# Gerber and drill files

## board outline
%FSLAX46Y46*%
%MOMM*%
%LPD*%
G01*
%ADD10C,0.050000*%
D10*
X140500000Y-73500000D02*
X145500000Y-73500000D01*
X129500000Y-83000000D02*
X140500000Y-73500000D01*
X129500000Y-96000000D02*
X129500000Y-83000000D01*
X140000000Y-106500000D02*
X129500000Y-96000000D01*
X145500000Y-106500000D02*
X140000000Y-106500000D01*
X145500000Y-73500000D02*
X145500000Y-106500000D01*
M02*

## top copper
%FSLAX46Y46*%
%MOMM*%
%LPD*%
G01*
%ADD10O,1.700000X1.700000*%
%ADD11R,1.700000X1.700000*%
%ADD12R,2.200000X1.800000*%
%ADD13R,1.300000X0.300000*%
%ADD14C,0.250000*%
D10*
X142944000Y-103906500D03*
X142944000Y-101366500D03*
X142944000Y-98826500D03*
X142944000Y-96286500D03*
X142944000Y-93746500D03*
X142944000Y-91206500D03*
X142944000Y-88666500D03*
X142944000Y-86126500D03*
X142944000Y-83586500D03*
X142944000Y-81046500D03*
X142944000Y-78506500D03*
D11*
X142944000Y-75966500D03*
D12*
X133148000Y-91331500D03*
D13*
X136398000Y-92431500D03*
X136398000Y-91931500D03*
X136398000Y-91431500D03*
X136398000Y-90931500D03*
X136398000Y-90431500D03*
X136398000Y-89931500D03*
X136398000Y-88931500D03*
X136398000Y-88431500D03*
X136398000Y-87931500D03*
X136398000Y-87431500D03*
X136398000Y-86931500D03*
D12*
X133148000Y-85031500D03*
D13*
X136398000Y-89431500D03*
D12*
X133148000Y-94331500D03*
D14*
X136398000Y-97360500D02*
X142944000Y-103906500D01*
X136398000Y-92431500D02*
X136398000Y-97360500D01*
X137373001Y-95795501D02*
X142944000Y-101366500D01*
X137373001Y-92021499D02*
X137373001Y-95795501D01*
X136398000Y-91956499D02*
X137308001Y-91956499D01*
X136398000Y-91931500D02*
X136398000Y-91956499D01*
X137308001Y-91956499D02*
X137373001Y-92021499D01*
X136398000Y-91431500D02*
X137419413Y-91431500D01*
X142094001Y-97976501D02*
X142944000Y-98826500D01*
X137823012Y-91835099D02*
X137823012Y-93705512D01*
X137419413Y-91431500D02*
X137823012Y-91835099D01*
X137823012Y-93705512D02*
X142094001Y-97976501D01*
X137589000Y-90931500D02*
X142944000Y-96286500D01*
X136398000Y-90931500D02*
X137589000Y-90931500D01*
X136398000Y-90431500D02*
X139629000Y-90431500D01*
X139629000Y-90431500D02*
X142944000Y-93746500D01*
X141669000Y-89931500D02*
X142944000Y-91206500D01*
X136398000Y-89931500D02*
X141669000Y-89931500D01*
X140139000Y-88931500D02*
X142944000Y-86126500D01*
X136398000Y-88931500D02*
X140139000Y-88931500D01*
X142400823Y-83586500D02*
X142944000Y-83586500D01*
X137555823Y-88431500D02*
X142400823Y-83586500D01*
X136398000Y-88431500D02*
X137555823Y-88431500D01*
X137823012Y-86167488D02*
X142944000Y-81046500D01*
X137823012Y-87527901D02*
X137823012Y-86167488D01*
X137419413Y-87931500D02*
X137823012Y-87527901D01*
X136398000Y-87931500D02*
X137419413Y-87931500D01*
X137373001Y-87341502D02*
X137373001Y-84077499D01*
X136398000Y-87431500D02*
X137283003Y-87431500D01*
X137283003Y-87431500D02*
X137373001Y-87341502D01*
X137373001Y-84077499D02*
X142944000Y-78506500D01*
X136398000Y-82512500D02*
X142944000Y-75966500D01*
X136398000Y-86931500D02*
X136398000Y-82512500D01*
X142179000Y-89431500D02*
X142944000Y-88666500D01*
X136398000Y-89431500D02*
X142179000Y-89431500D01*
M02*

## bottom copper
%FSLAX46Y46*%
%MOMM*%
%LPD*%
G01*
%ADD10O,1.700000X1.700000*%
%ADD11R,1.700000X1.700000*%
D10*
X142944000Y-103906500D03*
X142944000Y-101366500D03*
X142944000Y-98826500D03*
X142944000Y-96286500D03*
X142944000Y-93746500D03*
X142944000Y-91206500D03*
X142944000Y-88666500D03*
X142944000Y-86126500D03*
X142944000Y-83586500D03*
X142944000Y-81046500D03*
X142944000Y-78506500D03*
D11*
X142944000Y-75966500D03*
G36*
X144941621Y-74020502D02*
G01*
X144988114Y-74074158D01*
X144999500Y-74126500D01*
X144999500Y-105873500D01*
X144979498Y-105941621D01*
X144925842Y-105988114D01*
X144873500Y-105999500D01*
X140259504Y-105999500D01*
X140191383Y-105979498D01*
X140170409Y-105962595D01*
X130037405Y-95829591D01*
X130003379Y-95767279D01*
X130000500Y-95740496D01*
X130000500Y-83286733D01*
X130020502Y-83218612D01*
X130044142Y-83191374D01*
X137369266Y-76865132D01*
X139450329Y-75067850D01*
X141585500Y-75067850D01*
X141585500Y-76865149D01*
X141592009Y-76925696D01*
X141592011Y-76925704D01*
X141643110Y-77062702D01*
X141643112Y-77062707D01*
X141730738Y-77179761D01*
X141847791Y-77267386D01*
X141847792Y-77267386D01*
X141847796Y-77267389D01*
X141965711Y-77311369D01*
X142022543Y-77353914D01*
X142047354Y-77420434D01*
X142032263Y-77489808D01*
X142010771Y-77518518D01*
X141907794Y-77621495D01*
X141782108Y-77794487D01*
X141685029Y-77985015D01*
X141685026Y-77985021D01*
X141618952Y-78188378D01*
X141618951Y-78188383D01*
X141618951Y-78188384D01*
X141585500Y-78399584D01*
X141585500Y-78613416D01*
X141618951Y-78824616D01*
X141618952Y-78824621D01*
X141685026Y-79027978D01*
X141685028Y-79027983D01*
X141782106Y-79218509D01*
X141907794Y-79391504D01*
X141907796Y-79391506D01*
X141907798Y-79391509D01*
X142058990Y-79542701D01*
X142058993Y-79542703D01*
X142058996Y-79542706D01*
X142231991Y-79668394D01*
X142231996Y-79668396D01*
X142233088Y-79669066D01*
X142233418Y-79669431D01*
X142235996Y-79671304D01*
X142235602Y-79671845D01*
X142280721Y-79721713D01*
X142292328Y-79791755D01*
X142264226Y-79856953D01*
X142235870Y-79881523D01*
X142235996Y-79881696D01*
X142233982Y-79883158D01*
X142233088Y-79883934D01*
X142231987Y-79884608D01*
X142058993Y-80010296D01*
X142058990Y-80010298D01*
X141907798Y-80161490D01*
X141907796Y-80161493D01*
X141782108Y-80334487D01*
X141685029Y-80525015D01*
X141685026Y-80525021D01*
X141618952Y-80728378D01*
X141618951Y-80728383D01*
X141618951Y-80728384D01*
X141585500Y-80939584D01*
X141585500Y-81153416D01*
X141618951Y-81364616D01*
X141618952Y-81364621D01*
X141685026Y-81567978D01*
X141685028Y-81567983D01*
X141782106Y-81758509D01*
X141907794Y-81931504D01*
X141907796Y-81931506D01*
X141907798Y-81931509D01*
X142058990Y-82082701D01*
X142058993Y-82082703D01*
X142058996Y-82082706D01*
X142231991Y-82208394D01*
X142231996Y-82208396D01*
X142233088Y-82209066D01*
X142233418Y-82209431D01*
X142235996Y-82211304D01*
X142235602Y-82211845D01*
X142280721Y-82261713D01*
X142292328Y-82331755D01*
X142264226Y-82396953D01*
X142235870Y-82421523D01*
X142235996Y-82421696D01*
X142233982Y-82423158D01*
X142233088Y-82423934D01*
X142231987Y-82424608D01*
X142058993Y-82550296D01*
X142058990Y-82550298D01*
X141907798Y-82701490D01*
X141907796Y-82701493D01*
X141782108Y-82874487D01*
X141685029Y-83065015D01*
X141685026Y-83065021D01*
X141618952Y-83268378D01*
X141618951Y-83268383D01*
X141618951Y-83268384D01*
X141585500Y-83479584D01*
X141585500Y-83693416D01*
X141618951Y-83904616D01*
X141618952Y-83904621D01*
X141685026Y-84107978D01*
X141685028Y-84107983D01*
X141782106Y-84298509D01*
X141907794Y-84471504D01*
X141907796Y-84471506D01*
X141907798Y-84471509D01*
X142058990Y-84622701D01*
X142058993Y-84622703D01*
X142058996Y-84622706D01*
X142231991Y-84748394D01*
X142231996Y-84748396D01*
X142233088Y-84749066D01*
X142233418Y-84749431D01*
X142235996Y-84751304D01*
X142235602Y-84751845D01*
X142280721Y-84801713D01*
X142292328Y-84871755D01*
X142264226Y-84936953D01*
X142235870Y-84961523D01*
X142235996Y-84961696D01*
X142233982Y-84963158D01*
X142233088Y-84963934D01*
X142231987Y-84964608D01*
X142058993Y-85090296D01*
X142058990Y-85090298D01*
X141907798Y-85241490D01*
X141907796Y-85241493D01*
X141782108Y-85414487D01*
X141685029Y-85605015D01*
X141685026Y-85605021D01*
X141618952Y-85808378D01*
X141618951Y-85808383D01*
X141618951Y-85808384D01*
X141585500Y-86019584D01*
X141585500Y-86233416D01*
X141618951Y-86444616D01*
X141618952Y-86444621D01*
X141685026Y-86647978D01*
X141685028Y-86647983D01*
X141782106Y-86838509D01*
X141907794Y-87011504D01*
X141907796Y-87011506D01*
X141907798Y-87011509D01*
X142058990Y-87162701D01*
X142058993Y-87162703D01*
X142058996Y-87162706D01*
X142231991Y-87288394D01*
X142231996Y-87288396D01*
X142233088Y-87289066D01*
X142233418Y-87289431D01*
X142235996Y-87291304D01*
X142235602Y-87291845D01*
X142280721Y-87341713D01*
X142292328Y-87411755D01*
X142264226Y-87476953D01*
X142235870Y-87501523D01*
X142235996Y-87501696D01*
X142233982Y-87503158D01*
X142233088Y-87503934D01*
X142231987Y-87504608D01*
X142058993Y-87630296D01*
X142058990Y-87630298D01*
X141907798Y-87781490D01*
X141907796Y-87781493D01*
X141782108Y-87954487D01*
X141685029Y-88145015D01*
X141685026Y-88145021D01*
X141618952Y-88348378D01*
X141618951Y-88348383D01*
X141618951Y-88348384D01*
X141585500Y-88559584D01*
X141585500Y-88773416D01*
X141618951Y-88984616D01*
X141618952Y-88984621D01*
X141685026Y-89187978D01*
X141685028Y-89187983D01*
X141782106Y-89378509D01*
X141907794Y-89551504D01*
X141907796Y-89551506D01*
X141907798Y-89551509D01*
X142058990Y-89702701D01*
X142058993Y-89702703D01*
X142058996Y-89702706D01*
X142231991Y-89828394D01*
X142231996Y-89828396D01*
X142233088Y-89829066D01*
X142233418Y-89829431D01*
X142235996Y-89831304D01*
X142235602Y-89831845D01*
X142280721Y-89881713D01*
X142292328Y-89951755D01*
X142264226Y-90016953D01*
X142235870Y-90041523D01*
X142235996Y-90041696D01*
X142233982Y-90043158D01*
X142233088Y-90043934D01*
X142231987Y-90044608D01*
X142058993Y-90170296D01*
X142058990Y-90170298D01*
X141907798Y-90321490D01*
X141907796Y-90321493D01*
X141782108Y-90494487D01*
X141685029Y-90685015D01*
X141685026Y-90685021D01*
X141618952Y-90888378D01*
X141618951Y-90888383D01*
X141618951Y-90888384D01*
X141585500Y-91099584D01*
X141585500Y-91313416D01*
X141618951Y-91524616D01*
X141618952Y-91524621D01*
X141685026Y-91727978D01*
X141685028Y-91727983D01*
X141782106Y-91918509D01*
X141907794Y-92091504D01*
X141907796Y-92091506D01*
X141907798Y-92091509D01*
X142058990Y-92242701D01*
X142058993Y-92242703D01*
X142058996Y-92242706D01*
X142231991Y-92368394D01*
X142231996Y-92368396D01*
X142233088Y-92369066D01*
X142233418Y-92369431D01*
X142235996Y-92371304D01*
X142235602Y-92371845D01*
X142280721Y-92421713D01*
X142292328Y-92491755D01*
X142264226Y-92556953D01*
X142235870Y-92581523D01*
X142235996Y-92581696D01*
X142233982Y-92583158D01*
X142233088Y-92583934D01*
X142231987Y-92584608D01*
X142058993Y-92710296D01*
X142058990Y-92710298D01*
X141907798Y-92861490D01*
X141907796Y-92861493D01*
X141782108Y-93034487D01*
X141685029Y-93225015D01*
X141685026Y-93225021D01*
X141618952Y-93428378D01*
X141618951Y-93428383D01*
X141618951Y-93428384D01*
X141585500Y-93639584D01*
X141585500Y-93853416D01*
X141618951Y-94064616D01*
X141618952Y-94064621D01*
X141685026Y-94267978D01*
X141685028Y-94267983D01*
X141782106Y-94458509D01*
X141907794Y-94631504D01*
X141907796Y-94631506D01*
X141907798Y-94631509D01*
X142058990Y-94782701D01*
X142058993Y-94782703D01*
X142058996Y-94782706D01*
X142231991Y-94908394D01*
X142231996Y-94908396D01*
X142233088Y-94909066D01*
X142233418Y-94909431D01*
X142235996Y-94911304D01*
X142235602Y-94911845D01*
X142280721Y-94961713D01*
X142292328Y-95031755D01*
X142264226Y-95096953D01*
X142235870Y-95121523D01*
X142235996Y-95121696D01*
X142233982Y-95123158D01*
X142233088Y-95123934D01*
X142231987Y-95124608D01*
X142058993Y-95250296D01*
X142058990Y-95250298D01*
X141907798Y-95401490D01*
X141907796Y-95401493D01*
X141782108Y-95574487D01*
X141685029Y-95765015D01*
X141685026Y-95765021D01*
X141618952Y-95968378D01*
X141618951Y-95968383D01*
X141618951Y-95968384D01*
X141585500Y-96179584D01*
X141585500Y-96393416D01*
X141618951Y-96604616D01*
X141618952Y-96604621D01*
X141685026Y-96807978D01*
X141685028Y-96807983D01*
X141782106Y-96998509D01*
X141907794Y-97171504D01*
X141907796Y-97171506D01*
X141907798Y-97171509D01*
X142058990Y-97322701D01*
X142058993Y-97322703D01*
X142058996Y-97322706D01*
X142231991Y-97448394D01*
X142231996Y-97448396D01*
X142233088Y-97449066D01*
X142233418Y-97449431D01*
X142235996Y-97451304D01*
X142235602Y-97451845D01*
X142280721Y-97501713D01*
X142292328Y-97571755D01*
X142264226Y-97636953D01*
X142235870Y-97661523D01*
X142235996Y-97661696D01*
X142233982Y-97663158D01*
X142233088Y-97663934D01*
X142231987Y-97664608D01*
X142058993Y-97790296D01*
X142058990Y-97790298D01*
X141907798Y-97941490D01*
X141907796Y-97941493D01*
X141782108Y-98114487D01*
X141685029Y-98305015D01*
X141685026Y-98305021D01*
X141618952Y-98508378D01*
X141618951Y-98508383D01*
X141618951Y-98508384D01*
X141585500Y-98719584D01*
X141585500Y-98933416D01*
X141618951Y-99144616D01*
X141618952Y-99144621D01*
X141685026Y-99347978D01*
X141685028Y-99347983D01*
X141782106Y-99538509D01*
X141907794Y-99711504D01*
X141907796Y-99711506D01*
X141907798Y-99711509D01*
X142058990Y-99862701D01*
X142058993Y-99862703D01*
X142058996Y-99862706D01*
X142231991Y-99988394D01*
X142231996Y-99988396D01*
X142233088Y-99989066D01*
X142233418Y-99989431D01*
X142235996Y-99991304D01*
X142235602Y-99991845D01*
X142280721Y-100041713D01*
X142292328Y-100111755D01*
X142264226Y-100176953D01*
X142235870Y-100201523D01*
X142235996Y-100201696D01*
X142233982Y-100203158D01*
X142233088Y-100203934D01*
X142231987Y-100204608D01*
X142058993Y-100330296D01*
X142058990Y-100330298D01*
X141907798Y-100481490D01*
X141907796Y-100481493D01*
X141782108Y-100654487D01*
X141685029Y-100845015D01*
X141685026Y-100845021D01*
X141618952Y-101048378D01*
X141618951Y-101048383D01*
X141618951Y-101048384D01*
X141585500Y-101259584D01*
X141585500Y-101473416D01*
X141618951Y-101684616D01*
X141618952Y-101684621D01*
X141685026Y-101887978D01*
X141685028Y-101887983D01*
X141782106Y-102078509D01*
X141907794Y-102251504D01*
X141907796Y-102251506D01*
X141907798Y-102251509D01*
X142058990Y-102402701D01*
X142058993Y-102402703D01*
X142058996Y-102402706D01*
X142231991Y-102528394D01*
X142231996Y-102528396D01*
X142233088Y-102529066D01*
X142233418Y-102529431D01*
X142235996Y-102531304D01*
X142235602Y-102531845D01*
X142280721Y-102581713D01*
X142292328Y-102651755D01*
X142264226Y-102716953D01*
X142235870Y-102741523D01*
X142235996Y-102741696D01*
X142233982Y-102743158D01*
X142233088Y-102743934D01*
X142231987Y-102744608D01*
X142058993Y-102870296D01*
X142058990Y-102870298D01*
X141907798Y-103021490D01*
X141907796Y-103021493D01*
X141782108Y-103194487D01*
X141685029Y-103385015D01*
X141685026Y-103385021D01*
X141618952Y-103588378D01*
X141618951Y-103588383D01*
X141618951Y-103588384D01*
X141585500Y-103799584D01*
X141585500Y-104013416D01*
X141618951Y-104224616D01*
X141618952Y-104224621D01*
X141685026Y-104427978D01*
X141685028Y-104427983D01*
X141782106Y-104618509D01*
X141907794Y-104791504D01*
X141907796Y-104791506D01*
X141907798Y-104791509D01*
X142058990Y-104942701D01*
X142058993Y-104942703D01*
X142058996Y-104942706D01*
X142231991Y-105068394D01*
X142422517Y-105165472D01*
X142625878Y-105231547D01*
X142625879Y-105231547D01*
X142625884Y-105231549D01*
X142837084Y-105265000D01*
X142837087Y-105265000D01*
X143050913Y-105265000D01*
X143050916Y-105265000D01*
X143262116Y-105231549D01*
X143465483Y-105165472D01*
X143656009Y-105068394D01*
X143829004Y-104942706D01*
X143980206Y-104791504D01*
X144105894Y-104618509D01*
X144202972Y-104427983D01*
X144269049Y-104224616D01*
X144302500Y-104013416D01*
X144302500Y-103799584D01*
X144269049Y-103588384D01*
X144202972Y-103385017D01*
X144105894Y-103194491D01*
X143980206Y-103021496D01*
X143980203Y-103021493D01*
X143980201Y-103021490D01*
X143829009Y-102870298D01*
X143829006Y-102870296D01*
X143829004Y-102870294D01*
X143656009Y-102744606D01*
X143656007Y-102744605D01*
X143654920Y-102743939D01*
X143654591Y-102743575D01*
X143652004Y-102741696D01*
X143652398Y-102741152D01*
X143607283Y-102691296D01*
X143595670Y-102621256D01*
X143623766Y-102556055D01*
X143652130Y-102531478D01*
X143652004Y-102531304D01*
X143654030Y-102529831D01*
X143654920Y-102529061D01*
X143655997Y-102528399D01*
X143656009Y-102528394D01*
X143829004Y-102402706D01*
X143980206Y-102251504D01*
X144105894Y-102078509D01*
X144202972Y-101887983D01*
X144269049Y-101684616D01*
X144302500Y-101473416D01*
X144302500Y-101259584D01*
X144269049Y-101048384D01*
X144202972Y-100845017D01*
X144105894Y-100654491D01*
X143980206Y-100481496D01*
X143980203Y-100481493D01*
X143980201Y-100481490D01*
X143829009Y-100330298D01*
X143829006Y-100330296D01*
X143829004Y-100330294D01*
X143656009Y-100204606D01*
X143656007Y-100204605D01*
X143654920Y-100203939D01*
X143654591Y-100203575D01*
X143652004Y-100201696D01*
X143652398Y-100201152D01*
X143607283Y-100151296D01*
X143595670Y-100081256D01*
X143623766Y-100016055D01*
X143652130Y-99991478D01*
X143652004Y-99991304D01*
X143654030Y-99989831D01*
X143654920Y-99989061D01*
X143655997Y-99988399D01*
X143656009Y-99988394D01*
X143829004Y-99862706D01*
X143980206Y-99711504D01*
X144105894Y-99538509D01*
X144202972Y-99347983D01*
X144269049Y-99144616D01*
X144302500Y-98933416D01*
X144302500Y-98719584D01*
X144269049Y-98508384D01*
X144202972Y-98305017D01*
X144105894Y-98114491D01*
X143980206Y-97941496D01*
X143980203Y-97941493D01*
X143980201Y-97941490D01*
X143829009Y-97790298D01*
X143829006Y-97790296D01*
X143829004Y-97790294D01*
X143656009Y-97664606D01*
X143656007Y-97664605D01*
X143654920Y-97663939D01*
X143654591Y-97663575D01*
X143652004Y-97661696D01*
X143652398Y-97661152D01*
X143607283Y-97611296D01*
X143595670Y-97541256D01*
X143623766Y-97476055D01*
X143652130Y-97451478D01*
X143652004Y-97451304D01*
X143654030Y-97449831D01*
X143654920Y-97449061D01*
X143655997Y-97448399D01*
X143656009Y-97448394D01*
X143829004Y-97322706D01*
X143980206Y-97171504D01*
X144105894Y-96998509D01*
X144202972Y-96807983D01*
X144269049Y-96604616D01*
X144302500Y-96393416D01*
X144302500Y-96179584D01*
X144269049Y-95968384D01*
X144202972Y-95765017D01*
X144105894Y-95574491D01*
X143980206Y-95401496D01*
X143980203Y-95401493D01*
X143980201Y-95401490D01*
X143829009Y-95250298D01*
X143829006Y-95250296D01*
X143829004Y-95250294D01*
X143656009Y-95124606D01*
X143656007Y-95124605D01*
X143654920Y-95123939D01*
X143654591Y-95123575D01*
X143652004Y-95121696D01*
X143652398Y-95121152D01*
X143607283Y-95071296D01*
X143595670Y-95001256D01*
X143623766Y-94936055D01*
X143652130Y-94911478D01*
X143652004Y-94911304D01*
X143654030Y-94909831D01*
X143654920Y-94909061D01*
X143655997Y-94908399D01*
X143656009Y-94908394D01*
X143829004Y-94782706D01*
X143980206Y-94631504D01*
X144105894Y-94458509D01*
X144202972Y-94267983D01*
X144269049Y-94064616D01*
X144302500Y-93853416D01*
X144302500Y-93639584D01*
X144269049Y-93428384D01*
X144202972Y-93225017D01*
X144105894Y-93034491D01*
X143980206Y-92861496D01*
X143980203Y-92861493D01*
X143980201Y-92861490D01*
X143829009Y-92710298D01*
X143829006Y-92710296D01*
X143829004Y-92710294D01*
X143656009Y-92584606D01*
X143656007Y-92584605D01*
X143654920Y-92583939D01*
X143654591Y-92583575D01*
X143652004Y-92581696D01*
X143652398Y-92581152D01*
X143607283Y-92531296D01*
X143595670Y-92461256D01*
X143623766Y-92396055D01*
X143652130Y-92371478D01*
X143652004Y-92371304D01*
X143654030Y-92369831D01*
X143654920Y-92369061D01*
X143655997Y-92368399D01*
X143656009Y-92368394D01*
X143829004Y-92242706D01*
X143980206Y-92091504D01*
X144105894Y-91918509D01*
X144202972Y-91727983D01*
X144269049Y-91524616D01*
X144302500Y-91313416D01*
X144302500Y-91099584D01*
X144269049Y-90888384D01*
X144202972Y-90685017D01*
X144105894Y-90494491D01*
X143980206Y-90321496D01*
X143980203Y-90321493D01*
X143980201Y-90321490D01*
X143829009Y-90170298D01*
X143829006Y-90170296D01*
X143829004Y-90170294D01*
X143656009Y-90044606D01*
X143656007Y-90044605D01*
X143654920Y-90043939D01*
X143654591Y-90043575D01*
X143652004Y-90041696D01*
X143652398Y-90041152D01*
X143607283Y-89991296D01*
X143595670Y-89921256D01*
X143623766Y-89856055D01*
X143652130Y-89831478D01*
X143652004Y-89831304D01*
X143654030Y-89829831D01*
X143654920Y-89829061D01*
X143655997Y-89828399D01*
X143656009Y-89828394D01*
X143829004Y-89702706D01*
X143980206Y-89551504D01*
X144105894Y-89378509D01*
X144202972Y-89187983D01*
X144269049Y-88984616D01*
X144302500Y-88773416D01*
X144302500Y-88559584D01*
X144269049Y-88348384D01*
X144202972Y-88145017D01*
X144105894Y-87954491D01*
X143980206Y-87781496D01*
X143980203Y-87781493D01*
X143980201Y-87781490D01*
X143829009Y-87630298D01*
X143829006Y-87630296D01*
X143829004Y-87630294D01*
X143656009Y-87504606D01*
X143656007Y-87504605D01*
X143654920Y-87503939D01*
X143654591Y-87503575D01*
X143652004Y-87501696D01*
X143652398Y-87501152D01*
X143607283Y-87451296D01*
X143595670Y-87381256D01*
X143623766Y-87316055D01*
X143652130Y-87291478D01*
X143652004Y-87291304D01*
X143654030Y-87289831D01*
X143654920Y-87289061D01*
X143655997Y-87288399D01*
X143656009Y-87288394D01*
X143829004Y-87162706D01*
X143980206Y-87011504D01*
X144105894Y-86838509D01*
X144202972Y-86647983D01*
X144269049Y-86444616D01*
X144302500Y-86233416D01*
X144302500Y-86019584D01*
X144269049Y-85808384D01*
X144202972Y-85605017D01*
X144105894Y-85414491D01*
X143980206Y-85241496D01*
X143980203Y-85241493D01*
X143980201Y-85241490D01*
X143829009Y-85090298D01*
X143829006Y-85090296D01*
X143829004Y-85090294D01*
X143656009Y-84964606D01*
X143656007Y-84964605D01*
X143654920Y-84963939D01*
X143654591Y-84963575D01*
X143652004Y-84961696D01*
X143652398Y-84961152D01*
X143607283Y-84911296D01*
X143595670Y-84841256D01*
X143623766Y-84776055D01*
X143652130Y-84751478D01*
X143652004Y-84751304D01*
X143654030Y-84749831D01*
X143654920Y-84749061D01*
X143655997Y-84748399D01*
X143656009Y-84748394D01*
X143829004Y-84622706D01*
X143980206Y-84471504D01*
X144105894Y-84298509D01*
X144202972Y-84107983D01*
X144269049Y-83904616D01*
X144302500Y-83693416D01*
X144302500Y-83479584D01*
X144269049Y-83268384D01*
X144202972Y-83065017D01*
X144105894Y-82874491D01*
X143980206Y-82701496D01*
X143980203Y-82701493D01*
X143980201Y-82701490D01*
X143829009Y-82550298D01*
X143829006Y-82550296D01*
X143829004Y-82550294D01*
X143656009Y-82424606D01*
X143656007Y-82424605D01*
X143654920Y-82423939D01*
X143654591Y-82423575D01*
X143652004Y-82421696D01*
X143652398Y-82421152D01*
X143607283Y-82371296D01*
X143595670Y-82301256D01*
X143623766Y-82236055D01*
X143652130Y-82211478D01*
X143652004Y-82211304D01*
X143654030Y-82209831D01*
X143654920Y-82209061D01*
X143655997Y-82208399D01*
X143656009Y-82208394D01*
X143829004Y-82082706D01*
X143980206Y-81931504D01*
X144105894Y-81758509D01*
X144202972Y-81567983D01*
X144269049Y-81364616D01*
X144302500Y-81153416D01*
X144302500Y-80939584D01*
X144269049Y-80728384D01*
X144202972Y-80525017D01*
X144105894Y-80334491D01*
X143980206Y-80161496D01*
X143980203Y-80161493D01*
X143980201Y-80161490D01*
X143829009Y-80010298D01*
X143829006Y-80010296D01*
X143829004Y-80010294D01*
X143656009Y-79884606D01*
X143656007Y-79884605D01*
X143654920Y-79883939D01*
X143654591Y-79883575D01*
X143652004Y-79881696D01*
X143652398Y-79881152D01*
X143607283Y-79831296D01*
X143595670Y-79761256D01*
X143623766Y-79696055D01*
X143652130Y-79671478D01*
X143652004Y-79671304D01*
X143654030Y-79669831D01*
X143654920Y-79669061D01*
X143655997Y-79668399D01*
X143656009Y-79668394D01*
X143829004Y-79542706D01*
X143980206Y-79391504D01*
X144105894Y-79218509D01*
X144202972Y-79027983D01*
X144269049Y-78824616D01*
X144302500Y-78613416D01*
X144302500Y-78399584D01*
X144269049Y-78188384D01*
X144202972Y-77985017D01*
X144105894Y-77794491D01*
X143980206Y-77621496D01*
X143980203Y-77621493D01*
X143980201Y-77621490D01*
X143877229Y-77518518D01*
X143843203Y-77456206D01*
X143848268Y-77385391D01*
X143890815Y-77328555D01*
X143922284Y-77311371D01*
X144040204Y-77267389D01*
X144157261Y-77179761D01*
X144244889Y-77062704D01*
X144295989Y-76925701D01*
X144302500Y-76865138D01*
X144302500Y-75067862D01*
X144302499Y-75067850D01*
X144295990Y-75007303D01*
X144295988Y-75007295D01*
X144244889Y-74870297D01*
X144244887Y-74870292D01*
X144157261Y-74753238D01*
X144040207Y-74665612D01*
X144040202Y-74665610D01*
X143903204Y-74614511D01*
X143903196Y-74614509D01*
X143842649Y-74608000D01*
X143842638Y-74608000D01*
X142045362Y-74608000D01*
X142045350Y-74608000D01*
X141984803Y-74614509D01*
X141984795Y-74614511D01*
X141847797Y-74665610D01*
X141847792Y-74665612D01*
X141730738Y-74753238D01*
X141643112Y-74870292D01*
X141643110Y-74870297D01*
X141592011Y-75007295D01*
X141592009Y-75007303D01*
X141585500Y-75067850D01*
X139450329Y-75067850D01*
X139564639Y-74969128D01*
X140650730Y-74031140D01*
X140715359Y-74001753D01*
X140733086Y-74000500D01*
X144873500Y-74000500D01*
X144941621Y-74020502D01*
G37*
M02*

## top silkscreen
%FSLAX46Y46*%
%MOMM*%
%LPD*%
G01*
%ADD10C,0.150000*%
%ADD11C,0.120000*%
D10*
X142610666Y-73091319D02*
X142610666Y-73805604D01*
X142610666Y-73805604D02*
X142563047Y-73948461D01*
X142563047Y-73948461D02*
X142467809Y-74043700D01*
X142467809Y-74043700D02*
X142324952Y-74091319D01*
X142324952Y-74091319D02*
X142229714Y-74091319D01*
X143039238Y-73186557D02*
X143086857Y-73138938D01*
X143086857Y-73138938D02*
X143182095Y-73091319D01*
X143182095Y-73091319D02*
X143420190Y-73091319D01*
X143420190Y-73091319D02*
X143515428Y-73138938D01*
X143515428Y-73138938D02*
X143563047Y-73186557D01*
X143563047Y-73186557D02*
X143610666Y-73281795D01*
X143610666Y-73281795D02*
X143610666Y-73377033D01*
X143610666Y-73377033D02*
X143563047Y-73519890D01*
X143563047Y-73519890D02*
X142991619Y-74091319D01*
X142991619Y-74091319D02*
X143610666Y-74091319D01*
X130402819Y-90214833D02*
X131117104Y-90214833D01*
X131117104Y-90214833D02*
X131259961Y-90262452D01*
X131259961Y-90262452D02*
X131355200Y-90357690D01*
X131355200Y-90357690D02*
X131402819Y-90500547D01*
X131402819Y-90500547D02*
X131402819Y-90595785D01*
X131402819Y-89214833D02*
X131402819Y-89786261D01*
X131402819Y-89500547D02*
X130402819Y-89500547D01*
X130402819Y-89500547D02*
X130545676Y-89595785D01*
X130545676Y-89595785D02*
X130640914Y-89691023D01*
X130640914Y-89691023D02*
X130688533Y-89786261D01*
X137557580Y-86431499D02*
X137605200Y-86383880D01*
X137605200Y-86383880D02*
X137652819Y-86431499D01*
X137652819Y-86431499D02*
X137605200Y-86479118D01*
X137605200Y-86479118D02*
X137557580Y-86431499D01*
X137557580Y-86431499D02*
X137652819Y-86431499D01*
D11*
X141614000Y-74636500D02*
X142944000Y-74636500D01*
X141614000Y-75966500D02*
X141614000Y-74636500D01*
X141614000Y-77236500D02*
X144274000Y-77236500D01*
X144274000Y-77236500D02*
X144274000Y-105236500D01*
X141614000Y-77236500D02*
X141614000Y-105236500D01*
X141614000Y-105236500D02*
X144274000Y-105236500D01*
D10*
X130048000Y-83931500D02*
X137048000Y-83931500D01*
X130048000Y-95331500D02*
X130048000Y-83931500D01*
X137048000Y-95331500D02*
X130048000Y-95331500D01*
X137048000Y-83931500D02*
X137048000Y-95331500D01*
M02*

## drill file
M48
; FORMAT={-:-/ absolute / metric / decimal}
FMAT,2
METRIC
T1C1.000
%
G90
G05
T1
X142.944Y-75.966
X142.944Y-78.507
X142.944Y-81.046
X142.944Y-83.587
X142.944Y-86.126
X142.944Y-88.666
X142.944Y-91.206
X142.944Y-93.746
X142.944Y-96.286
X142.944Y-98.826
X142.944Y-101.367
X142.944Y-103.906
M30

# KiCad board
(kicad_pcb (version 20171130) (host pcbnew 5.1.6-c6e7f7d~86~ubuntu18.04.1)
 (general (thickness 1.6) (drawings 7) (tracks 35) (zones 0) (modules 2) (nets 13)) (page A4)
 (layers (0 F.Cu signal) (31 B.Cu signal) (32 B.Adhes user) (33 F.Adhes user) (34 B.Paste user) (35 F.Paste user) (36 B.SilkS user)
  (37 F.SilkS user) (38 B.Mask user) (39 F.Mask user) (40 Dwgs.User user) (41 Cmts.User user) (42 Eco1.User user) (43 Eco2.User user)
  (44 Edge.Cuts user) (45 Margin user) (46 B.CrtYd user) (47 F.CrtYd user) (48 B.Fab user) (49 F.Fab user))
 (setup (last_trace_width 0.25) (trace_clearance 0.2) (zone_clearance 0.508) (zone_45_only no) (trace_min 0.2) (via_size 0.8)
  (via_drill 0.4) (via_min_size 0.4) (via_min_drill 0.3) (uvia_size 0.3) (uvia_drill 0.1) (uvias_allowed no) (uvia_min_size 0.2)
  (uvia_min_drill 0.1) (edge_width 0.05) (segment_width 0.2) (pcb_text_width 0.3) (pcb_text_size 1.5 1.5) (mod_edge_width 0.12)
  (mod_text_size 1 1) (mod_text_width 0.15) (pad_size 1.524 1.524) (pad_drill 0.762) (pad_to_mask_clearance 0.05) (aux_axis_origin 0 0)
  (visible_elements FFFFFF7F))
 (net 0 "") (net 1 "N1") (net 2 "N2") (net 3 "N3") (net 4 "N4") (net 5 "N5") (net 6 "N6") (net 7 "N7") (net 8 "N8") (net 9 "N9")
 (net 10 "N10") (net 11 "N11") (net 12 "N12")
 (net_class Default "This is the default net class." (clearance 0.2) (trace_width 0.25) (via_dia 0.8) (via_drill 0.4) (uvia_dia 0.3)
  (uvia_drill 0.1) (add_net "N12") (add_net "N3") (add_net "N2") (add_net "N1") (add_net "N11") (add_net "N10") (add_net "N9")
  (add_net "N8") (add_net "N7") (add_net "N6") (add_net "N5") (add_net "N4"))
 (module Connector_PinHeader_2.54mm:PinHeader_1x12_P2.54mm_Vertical (layer F.Cu) (at 142.944 75.9665)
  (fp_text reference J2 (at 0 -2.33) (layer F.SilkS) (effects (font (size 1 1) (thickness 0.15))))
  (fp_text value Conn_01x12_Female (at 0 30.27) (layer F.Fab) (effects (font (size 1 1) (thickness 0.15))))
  (fp_line (start -1.33 -1.33) (end 0 -1.33) (layer F.SilkS) (width 0.12))
  (fp_line (start -1.33 0) (end -1.33 -1.33) (layer F.SilkS) (width 0.12))
  (fp_line (start -1.33 1.27) (end 1.33 1.27) (layer F.SilkS) (width 0.12))
  (fp_line (start 1.33 1.27) (end 1.33 29.27) (layer F.SilkS) (width 0.12))
  (fp_line (start -1.33 1.27) (end -1.33 29.27) (layer F.SilkS) (width 0.12))
  (fp_line (start -1.33 29.27) (end 1.33 29.27) (layer F.SilkS) (width 0.12))
  (pad 12 thru_hole oval (at 0 27.94) (size 1.7 1.7) (drill 1) (layers *.Cu *.Mask) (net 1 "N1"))
  (pad 11 thru_hole oval (at 0 25.4) (size 1.7 1.7) (drill 1) (layers *.Cu *.Mask) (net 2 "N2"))
  (pad 10 thru_hole oval (at 0 22.86) (size 1.7 1.7) (drill 1) (layers *.Cu *.Mask) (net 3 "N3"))
  (pad 9 thru_hole oval (at 0 20.32) (size 1.7 1.7) (drill 1) (layers *.Cu *.Mask) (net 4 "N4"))
  (pad 8 thru_hole oval (at 0 17.78) (size 1.7 1.7) (drill 1) (layers *.Cu *.Mask) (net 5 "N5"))
  (pad 7 thru_hole oval (at 0 15.24) (size 1.7 1.7) (drill 1) (layers *.Cu *.Mask) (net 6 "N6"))
  (pad 6 thru_hole oval (at 0 12.7) (size 1.7 1.7) (drill 1) (layers *.Cu *.Mask) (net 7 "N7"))
  (pad 5 thru_hole oval (at 0 10.16) (size 1.7 1.7) (drill 1) (layers *.Cu *.Mask) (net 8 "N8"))
  (pad 4 thru_hole oval (at 0 7.62) (size 1.7 1.7) (drill 1) (layers *.Cu *.Mask) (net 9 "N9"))
  (pad 3 thru_hole oval (at 0 5.08) (size 1.7 1.7) (drill 1) (layers *.Cu *.Mask) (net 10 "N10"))
  (pad 2 thru_hole oval (at 0 2.54) (size 1.7 1.7) (drill 1) (layers *.Cu *.Mask) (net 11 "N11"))
  (pad 1 thru_hole rect (at 0 0) (size 1.7 1.7) (drill 1) (layers *.Cu *.Mask) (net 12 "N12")))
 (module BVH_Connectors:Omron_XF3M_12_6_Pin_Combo (layer F.Cu) (at 136.398 86.9315 270)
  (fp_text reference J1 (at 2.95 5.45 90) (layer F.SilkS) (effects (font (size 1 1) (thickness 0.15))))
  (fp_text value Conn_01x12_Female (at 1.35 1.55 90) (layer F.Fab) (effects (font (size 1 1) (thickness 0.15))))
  (fp_line (start -3 6.35) (end -3 -0.65) (layer F.SilkS) (width 0.15))
  (fp_line (start 8.4 6.35) (end -3 6.35) (layer F.SilkS) (width 0.15))
  (fp_line (start 8.4 -0.65) (end 8.4 6.35) (layer F.SilkS) (width 0.15))
  (fp_line (start -3 -0.65) (end 8.4 -0.65) (layer F.SilkS) (width 0.15))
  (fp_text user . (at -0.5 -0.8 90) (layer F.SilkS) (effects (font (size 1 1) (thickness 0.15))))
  (pad "" smd rect (at 4.4 3.25 270) (size 1.8 2.2) (layers F.Cu F.Paste F.Mask))
  (pad 12 smd rect (at 5.5 0 270) (size 0.3 1.3) (layers F.Cu F.Paste F.Mask) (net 1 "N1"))
  (pad 11 smd rect (at 5 0 270) (size 0.3 1.3) (layers F.Cu F.Paste F.Mask) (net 2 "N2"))
  (pad 10 smd rect (at 4.5 0 270) (size 0.3 1.3) (layers F.Cu F.Paste F.Mask) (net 3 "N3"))
  (pad 9 smd rect (at 4 0 270) (size 0.3 1.3) (layers F.Cu F.Paste F.Mask) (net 4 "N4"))
  (pad 8 smd rect (at 3.5 0 270) (size 0.3 1.3) (layers F.Cu F.Paste F.Mask) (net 5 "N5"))
  (pad 7 smd rect (at 3 0 270) (size 0.3 1.3) (layers F.Cu F.Paste F.Mask) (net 6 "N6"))
  (pad 5 smd rect (at 2 0 270) (size 0.3 1.3) (layers F.Cu F.Paste F.Mask) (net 8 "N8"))
  (pad 4 smd rect (at 1.5 0 270) (size 0.3 1.3) (layers F.Cu F.Paste F.Mask) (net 9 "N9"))
  (pad 3 smd rect (at 1 0 270) (size 0.3 1.3) (layers F.Cu F.Paste F.Mask) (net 10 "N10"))
  (pad 2 smd rect (at 0.5 0 270) (size 0.3 1.3) (layers F.Cu F.Paste F.Mask) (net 11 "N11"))
  (pad 1 smd rect (at 0 0 270) (size 0.3 1.3) (layers F.Cu F.Paste F.Mask) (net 12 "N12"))
  (pad "" smd rect (at -1.9 3.25 270) (size 1.8 2.2) (layers F.Cu F.Paste F.Mask))
  (pad 6 smd rect (at 2.5 0 270) (size 0.3 1.3) (layers F.Cu F.Paste F.Mask) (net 7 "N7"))
  (pad "" smd rect (at 7.4 3.25 270) (size 1.8 2.2) (layers F.Cu F.Paste F.Mask)))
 (gr_line (start 140.5 73.5) (end 145.5 73.5) (layer Edge.Cuts) (width 0.05))
 (gr_line (start 129.5 83) (end 140.5 73.5) (layer Edge.Cuts) (width 0.05))
 (gr_line (start 129.5 96) (end 129.5 83) (layer Edge.Cuts) (width 0.05))
 (gr_line (start 140 106.5) (end 129.5 96) (layer Edge.Cuts) (width 0.05))
 (gr_line (start 145.5 106.5) (end 140 106.5) (layer Edge.Cuts) (width 0.05))
 (gr_line (start 145.5 73.5) (end 145.5 106.5) (layer Edge.Cuts) (width 0.05))
 (segment (start 136.398 97.3605) (end 142.944 103.9065) (width 0.25) (layer F.Cu) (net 1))
 (segment (start 136.398 92.4315) (end 136.398 97.3605) (width 0.25) (layer F.Cu) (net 1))
 (segment (start 137.373001 95.795501) (end 142.944 101.3665) (width 0.25) (layer F.Cu) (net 2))
 (segment (start 137.373001 92.021499) (end 137.373001 95.795501) (width 0.25) (layer F.Cu) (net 2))
 (segment (start 136.398 91.956499) (end 137.308001 91.956499) (width 0.25) (layer F.Cu) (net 2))
 (segment (start 136.398 91.9315) (end 136.398 91.956499) (width 0.25) (layer F.Cu) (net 2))
 (segment (start 137.308001 91.956499) (end 137.373001 92.021499) (width 0.25) (layer F.Cu) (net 2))
 (segment (start 136.398 91.4315) (end 137.419413 91.4315) (width 0.25) (layer F.Cu) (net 3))
 (segment (start 142.094001 97.976501) (end 142.944 98.8265) (width 0.25) (layer F.Cu) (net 3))
 (segment (start 137.823012 91.835099) (end 137.823012 93.705512) (width 0.25) (layer F.Cu) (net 3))
 (segment (start 137.419413 91.4315) (end 137.823012 91.835099) (width 0.25) (layer F.Cu) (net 3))
 (segment (start 137.823012 93.705512) (end 142.094001 97.976501) (width 0.25) (layer F.Cu) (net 3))
 (segment (start 137.589 90.9315) (end 142.944 96.2865) (width 0.25) (layer F.Cu) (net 4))
 (segment (start 136.398 90.9315) (end 137.589 90.9315) (width 0.25) (layer F.Cu) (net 4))
 (segment (start 136.398 90.4315) (end 139.629 90.4315) (width 0.25) (layer F.Cu) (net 5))
 (segment (start 139.629 90.4315) (end 142.944 93.7465) (width 0.25) (layer F.Cu) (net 5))
 (segment (start 141.669 89.9315) (end 142.944 91.2065) (width 0.25) (layer F.Cu) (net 6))
 (segment (start 136.398 89.9315) (end 141.669 89.9315) (width 0.25) (layer F.Cu) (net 6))
 (segment (start 140.139 88.9315) (end 142.944 86.1265) (width 0.25) (layer F.Cu) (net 8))
 (segment (start 136.398 88.9315) (end 140.139 88.9315) (width 0.25) (layer F.Cu) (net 8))
 (segment (start 142.400823 83.5865) (end 142.944 83.5865) (width 0.25) (layer F.Cu) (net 9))
 (segment (start 137.555823 88.4315) (end 142.400823 83.5865) (width 0.25) (layer F.Cu) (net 9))
 (segment (start 136.398 88.4315) (end 137.555823 88.4315) (width 0.25) (layer F.Cu) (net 9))
 (segment (start 137.823012 86.167488) (end 142.944 81.0465) (width 0.25) (layer F.Cu) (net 10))
 (segment (start 137.823012 87.527901) (end 137.823012 86.167488) (width 0.25) (layer F.Cu) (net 10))
 (segment (start 137.419413 87.9315) (end 137.823012 87.527901) (width 0.25) (layer F.Cu) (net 10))
 (segment (start 136.398 87.9315) (end 137.419413 87.9315) (width 0.25) (layer F.Cu) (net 10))
 (segment (start 137.373001 87.341502) (end 137.373001 84.077499) (width 0.25) (layer F.Cu) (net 11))
 (segment (start 136.398 87.4315) (end 137.283003 87.4315) (width 0.25) (layer F.Cu) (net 11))
 (segment (start 137.283003 87.4315) (end 137.373001 87.341502) (width 0.25) (layer F.Cu) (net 11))
 (segment (start 137.373001 84.077499) (end 142.944 78.5065) (width 0.25) (layer F.Cu) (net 11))
 (segment (start 136.398 82.5125) (end 142.944 75.9665) (width 0.25) (layer F.Cu) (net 12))
 (segment (start 136.398 86.9315) (end 136.398 82.5125) (width 0.25) (layer F.Cu) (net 12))
 (segment (start 142.179 89.4315) (end 142.944 88.6665) (width 0.25) (layer F.Cu) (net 7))
 (segment (start 136.398 89.4315) (end 142.179 89.4315) (width 0.25) (layer F.Cu) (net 7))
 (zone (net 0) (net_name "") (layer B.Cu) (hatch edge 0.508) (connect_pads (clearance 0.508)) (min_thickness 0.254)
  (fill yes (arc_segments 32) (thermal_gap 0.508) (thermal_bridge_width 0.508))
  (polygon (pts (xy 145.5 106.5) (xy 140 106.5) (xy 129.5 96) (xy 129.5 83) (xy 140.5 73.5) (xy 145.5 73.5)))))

